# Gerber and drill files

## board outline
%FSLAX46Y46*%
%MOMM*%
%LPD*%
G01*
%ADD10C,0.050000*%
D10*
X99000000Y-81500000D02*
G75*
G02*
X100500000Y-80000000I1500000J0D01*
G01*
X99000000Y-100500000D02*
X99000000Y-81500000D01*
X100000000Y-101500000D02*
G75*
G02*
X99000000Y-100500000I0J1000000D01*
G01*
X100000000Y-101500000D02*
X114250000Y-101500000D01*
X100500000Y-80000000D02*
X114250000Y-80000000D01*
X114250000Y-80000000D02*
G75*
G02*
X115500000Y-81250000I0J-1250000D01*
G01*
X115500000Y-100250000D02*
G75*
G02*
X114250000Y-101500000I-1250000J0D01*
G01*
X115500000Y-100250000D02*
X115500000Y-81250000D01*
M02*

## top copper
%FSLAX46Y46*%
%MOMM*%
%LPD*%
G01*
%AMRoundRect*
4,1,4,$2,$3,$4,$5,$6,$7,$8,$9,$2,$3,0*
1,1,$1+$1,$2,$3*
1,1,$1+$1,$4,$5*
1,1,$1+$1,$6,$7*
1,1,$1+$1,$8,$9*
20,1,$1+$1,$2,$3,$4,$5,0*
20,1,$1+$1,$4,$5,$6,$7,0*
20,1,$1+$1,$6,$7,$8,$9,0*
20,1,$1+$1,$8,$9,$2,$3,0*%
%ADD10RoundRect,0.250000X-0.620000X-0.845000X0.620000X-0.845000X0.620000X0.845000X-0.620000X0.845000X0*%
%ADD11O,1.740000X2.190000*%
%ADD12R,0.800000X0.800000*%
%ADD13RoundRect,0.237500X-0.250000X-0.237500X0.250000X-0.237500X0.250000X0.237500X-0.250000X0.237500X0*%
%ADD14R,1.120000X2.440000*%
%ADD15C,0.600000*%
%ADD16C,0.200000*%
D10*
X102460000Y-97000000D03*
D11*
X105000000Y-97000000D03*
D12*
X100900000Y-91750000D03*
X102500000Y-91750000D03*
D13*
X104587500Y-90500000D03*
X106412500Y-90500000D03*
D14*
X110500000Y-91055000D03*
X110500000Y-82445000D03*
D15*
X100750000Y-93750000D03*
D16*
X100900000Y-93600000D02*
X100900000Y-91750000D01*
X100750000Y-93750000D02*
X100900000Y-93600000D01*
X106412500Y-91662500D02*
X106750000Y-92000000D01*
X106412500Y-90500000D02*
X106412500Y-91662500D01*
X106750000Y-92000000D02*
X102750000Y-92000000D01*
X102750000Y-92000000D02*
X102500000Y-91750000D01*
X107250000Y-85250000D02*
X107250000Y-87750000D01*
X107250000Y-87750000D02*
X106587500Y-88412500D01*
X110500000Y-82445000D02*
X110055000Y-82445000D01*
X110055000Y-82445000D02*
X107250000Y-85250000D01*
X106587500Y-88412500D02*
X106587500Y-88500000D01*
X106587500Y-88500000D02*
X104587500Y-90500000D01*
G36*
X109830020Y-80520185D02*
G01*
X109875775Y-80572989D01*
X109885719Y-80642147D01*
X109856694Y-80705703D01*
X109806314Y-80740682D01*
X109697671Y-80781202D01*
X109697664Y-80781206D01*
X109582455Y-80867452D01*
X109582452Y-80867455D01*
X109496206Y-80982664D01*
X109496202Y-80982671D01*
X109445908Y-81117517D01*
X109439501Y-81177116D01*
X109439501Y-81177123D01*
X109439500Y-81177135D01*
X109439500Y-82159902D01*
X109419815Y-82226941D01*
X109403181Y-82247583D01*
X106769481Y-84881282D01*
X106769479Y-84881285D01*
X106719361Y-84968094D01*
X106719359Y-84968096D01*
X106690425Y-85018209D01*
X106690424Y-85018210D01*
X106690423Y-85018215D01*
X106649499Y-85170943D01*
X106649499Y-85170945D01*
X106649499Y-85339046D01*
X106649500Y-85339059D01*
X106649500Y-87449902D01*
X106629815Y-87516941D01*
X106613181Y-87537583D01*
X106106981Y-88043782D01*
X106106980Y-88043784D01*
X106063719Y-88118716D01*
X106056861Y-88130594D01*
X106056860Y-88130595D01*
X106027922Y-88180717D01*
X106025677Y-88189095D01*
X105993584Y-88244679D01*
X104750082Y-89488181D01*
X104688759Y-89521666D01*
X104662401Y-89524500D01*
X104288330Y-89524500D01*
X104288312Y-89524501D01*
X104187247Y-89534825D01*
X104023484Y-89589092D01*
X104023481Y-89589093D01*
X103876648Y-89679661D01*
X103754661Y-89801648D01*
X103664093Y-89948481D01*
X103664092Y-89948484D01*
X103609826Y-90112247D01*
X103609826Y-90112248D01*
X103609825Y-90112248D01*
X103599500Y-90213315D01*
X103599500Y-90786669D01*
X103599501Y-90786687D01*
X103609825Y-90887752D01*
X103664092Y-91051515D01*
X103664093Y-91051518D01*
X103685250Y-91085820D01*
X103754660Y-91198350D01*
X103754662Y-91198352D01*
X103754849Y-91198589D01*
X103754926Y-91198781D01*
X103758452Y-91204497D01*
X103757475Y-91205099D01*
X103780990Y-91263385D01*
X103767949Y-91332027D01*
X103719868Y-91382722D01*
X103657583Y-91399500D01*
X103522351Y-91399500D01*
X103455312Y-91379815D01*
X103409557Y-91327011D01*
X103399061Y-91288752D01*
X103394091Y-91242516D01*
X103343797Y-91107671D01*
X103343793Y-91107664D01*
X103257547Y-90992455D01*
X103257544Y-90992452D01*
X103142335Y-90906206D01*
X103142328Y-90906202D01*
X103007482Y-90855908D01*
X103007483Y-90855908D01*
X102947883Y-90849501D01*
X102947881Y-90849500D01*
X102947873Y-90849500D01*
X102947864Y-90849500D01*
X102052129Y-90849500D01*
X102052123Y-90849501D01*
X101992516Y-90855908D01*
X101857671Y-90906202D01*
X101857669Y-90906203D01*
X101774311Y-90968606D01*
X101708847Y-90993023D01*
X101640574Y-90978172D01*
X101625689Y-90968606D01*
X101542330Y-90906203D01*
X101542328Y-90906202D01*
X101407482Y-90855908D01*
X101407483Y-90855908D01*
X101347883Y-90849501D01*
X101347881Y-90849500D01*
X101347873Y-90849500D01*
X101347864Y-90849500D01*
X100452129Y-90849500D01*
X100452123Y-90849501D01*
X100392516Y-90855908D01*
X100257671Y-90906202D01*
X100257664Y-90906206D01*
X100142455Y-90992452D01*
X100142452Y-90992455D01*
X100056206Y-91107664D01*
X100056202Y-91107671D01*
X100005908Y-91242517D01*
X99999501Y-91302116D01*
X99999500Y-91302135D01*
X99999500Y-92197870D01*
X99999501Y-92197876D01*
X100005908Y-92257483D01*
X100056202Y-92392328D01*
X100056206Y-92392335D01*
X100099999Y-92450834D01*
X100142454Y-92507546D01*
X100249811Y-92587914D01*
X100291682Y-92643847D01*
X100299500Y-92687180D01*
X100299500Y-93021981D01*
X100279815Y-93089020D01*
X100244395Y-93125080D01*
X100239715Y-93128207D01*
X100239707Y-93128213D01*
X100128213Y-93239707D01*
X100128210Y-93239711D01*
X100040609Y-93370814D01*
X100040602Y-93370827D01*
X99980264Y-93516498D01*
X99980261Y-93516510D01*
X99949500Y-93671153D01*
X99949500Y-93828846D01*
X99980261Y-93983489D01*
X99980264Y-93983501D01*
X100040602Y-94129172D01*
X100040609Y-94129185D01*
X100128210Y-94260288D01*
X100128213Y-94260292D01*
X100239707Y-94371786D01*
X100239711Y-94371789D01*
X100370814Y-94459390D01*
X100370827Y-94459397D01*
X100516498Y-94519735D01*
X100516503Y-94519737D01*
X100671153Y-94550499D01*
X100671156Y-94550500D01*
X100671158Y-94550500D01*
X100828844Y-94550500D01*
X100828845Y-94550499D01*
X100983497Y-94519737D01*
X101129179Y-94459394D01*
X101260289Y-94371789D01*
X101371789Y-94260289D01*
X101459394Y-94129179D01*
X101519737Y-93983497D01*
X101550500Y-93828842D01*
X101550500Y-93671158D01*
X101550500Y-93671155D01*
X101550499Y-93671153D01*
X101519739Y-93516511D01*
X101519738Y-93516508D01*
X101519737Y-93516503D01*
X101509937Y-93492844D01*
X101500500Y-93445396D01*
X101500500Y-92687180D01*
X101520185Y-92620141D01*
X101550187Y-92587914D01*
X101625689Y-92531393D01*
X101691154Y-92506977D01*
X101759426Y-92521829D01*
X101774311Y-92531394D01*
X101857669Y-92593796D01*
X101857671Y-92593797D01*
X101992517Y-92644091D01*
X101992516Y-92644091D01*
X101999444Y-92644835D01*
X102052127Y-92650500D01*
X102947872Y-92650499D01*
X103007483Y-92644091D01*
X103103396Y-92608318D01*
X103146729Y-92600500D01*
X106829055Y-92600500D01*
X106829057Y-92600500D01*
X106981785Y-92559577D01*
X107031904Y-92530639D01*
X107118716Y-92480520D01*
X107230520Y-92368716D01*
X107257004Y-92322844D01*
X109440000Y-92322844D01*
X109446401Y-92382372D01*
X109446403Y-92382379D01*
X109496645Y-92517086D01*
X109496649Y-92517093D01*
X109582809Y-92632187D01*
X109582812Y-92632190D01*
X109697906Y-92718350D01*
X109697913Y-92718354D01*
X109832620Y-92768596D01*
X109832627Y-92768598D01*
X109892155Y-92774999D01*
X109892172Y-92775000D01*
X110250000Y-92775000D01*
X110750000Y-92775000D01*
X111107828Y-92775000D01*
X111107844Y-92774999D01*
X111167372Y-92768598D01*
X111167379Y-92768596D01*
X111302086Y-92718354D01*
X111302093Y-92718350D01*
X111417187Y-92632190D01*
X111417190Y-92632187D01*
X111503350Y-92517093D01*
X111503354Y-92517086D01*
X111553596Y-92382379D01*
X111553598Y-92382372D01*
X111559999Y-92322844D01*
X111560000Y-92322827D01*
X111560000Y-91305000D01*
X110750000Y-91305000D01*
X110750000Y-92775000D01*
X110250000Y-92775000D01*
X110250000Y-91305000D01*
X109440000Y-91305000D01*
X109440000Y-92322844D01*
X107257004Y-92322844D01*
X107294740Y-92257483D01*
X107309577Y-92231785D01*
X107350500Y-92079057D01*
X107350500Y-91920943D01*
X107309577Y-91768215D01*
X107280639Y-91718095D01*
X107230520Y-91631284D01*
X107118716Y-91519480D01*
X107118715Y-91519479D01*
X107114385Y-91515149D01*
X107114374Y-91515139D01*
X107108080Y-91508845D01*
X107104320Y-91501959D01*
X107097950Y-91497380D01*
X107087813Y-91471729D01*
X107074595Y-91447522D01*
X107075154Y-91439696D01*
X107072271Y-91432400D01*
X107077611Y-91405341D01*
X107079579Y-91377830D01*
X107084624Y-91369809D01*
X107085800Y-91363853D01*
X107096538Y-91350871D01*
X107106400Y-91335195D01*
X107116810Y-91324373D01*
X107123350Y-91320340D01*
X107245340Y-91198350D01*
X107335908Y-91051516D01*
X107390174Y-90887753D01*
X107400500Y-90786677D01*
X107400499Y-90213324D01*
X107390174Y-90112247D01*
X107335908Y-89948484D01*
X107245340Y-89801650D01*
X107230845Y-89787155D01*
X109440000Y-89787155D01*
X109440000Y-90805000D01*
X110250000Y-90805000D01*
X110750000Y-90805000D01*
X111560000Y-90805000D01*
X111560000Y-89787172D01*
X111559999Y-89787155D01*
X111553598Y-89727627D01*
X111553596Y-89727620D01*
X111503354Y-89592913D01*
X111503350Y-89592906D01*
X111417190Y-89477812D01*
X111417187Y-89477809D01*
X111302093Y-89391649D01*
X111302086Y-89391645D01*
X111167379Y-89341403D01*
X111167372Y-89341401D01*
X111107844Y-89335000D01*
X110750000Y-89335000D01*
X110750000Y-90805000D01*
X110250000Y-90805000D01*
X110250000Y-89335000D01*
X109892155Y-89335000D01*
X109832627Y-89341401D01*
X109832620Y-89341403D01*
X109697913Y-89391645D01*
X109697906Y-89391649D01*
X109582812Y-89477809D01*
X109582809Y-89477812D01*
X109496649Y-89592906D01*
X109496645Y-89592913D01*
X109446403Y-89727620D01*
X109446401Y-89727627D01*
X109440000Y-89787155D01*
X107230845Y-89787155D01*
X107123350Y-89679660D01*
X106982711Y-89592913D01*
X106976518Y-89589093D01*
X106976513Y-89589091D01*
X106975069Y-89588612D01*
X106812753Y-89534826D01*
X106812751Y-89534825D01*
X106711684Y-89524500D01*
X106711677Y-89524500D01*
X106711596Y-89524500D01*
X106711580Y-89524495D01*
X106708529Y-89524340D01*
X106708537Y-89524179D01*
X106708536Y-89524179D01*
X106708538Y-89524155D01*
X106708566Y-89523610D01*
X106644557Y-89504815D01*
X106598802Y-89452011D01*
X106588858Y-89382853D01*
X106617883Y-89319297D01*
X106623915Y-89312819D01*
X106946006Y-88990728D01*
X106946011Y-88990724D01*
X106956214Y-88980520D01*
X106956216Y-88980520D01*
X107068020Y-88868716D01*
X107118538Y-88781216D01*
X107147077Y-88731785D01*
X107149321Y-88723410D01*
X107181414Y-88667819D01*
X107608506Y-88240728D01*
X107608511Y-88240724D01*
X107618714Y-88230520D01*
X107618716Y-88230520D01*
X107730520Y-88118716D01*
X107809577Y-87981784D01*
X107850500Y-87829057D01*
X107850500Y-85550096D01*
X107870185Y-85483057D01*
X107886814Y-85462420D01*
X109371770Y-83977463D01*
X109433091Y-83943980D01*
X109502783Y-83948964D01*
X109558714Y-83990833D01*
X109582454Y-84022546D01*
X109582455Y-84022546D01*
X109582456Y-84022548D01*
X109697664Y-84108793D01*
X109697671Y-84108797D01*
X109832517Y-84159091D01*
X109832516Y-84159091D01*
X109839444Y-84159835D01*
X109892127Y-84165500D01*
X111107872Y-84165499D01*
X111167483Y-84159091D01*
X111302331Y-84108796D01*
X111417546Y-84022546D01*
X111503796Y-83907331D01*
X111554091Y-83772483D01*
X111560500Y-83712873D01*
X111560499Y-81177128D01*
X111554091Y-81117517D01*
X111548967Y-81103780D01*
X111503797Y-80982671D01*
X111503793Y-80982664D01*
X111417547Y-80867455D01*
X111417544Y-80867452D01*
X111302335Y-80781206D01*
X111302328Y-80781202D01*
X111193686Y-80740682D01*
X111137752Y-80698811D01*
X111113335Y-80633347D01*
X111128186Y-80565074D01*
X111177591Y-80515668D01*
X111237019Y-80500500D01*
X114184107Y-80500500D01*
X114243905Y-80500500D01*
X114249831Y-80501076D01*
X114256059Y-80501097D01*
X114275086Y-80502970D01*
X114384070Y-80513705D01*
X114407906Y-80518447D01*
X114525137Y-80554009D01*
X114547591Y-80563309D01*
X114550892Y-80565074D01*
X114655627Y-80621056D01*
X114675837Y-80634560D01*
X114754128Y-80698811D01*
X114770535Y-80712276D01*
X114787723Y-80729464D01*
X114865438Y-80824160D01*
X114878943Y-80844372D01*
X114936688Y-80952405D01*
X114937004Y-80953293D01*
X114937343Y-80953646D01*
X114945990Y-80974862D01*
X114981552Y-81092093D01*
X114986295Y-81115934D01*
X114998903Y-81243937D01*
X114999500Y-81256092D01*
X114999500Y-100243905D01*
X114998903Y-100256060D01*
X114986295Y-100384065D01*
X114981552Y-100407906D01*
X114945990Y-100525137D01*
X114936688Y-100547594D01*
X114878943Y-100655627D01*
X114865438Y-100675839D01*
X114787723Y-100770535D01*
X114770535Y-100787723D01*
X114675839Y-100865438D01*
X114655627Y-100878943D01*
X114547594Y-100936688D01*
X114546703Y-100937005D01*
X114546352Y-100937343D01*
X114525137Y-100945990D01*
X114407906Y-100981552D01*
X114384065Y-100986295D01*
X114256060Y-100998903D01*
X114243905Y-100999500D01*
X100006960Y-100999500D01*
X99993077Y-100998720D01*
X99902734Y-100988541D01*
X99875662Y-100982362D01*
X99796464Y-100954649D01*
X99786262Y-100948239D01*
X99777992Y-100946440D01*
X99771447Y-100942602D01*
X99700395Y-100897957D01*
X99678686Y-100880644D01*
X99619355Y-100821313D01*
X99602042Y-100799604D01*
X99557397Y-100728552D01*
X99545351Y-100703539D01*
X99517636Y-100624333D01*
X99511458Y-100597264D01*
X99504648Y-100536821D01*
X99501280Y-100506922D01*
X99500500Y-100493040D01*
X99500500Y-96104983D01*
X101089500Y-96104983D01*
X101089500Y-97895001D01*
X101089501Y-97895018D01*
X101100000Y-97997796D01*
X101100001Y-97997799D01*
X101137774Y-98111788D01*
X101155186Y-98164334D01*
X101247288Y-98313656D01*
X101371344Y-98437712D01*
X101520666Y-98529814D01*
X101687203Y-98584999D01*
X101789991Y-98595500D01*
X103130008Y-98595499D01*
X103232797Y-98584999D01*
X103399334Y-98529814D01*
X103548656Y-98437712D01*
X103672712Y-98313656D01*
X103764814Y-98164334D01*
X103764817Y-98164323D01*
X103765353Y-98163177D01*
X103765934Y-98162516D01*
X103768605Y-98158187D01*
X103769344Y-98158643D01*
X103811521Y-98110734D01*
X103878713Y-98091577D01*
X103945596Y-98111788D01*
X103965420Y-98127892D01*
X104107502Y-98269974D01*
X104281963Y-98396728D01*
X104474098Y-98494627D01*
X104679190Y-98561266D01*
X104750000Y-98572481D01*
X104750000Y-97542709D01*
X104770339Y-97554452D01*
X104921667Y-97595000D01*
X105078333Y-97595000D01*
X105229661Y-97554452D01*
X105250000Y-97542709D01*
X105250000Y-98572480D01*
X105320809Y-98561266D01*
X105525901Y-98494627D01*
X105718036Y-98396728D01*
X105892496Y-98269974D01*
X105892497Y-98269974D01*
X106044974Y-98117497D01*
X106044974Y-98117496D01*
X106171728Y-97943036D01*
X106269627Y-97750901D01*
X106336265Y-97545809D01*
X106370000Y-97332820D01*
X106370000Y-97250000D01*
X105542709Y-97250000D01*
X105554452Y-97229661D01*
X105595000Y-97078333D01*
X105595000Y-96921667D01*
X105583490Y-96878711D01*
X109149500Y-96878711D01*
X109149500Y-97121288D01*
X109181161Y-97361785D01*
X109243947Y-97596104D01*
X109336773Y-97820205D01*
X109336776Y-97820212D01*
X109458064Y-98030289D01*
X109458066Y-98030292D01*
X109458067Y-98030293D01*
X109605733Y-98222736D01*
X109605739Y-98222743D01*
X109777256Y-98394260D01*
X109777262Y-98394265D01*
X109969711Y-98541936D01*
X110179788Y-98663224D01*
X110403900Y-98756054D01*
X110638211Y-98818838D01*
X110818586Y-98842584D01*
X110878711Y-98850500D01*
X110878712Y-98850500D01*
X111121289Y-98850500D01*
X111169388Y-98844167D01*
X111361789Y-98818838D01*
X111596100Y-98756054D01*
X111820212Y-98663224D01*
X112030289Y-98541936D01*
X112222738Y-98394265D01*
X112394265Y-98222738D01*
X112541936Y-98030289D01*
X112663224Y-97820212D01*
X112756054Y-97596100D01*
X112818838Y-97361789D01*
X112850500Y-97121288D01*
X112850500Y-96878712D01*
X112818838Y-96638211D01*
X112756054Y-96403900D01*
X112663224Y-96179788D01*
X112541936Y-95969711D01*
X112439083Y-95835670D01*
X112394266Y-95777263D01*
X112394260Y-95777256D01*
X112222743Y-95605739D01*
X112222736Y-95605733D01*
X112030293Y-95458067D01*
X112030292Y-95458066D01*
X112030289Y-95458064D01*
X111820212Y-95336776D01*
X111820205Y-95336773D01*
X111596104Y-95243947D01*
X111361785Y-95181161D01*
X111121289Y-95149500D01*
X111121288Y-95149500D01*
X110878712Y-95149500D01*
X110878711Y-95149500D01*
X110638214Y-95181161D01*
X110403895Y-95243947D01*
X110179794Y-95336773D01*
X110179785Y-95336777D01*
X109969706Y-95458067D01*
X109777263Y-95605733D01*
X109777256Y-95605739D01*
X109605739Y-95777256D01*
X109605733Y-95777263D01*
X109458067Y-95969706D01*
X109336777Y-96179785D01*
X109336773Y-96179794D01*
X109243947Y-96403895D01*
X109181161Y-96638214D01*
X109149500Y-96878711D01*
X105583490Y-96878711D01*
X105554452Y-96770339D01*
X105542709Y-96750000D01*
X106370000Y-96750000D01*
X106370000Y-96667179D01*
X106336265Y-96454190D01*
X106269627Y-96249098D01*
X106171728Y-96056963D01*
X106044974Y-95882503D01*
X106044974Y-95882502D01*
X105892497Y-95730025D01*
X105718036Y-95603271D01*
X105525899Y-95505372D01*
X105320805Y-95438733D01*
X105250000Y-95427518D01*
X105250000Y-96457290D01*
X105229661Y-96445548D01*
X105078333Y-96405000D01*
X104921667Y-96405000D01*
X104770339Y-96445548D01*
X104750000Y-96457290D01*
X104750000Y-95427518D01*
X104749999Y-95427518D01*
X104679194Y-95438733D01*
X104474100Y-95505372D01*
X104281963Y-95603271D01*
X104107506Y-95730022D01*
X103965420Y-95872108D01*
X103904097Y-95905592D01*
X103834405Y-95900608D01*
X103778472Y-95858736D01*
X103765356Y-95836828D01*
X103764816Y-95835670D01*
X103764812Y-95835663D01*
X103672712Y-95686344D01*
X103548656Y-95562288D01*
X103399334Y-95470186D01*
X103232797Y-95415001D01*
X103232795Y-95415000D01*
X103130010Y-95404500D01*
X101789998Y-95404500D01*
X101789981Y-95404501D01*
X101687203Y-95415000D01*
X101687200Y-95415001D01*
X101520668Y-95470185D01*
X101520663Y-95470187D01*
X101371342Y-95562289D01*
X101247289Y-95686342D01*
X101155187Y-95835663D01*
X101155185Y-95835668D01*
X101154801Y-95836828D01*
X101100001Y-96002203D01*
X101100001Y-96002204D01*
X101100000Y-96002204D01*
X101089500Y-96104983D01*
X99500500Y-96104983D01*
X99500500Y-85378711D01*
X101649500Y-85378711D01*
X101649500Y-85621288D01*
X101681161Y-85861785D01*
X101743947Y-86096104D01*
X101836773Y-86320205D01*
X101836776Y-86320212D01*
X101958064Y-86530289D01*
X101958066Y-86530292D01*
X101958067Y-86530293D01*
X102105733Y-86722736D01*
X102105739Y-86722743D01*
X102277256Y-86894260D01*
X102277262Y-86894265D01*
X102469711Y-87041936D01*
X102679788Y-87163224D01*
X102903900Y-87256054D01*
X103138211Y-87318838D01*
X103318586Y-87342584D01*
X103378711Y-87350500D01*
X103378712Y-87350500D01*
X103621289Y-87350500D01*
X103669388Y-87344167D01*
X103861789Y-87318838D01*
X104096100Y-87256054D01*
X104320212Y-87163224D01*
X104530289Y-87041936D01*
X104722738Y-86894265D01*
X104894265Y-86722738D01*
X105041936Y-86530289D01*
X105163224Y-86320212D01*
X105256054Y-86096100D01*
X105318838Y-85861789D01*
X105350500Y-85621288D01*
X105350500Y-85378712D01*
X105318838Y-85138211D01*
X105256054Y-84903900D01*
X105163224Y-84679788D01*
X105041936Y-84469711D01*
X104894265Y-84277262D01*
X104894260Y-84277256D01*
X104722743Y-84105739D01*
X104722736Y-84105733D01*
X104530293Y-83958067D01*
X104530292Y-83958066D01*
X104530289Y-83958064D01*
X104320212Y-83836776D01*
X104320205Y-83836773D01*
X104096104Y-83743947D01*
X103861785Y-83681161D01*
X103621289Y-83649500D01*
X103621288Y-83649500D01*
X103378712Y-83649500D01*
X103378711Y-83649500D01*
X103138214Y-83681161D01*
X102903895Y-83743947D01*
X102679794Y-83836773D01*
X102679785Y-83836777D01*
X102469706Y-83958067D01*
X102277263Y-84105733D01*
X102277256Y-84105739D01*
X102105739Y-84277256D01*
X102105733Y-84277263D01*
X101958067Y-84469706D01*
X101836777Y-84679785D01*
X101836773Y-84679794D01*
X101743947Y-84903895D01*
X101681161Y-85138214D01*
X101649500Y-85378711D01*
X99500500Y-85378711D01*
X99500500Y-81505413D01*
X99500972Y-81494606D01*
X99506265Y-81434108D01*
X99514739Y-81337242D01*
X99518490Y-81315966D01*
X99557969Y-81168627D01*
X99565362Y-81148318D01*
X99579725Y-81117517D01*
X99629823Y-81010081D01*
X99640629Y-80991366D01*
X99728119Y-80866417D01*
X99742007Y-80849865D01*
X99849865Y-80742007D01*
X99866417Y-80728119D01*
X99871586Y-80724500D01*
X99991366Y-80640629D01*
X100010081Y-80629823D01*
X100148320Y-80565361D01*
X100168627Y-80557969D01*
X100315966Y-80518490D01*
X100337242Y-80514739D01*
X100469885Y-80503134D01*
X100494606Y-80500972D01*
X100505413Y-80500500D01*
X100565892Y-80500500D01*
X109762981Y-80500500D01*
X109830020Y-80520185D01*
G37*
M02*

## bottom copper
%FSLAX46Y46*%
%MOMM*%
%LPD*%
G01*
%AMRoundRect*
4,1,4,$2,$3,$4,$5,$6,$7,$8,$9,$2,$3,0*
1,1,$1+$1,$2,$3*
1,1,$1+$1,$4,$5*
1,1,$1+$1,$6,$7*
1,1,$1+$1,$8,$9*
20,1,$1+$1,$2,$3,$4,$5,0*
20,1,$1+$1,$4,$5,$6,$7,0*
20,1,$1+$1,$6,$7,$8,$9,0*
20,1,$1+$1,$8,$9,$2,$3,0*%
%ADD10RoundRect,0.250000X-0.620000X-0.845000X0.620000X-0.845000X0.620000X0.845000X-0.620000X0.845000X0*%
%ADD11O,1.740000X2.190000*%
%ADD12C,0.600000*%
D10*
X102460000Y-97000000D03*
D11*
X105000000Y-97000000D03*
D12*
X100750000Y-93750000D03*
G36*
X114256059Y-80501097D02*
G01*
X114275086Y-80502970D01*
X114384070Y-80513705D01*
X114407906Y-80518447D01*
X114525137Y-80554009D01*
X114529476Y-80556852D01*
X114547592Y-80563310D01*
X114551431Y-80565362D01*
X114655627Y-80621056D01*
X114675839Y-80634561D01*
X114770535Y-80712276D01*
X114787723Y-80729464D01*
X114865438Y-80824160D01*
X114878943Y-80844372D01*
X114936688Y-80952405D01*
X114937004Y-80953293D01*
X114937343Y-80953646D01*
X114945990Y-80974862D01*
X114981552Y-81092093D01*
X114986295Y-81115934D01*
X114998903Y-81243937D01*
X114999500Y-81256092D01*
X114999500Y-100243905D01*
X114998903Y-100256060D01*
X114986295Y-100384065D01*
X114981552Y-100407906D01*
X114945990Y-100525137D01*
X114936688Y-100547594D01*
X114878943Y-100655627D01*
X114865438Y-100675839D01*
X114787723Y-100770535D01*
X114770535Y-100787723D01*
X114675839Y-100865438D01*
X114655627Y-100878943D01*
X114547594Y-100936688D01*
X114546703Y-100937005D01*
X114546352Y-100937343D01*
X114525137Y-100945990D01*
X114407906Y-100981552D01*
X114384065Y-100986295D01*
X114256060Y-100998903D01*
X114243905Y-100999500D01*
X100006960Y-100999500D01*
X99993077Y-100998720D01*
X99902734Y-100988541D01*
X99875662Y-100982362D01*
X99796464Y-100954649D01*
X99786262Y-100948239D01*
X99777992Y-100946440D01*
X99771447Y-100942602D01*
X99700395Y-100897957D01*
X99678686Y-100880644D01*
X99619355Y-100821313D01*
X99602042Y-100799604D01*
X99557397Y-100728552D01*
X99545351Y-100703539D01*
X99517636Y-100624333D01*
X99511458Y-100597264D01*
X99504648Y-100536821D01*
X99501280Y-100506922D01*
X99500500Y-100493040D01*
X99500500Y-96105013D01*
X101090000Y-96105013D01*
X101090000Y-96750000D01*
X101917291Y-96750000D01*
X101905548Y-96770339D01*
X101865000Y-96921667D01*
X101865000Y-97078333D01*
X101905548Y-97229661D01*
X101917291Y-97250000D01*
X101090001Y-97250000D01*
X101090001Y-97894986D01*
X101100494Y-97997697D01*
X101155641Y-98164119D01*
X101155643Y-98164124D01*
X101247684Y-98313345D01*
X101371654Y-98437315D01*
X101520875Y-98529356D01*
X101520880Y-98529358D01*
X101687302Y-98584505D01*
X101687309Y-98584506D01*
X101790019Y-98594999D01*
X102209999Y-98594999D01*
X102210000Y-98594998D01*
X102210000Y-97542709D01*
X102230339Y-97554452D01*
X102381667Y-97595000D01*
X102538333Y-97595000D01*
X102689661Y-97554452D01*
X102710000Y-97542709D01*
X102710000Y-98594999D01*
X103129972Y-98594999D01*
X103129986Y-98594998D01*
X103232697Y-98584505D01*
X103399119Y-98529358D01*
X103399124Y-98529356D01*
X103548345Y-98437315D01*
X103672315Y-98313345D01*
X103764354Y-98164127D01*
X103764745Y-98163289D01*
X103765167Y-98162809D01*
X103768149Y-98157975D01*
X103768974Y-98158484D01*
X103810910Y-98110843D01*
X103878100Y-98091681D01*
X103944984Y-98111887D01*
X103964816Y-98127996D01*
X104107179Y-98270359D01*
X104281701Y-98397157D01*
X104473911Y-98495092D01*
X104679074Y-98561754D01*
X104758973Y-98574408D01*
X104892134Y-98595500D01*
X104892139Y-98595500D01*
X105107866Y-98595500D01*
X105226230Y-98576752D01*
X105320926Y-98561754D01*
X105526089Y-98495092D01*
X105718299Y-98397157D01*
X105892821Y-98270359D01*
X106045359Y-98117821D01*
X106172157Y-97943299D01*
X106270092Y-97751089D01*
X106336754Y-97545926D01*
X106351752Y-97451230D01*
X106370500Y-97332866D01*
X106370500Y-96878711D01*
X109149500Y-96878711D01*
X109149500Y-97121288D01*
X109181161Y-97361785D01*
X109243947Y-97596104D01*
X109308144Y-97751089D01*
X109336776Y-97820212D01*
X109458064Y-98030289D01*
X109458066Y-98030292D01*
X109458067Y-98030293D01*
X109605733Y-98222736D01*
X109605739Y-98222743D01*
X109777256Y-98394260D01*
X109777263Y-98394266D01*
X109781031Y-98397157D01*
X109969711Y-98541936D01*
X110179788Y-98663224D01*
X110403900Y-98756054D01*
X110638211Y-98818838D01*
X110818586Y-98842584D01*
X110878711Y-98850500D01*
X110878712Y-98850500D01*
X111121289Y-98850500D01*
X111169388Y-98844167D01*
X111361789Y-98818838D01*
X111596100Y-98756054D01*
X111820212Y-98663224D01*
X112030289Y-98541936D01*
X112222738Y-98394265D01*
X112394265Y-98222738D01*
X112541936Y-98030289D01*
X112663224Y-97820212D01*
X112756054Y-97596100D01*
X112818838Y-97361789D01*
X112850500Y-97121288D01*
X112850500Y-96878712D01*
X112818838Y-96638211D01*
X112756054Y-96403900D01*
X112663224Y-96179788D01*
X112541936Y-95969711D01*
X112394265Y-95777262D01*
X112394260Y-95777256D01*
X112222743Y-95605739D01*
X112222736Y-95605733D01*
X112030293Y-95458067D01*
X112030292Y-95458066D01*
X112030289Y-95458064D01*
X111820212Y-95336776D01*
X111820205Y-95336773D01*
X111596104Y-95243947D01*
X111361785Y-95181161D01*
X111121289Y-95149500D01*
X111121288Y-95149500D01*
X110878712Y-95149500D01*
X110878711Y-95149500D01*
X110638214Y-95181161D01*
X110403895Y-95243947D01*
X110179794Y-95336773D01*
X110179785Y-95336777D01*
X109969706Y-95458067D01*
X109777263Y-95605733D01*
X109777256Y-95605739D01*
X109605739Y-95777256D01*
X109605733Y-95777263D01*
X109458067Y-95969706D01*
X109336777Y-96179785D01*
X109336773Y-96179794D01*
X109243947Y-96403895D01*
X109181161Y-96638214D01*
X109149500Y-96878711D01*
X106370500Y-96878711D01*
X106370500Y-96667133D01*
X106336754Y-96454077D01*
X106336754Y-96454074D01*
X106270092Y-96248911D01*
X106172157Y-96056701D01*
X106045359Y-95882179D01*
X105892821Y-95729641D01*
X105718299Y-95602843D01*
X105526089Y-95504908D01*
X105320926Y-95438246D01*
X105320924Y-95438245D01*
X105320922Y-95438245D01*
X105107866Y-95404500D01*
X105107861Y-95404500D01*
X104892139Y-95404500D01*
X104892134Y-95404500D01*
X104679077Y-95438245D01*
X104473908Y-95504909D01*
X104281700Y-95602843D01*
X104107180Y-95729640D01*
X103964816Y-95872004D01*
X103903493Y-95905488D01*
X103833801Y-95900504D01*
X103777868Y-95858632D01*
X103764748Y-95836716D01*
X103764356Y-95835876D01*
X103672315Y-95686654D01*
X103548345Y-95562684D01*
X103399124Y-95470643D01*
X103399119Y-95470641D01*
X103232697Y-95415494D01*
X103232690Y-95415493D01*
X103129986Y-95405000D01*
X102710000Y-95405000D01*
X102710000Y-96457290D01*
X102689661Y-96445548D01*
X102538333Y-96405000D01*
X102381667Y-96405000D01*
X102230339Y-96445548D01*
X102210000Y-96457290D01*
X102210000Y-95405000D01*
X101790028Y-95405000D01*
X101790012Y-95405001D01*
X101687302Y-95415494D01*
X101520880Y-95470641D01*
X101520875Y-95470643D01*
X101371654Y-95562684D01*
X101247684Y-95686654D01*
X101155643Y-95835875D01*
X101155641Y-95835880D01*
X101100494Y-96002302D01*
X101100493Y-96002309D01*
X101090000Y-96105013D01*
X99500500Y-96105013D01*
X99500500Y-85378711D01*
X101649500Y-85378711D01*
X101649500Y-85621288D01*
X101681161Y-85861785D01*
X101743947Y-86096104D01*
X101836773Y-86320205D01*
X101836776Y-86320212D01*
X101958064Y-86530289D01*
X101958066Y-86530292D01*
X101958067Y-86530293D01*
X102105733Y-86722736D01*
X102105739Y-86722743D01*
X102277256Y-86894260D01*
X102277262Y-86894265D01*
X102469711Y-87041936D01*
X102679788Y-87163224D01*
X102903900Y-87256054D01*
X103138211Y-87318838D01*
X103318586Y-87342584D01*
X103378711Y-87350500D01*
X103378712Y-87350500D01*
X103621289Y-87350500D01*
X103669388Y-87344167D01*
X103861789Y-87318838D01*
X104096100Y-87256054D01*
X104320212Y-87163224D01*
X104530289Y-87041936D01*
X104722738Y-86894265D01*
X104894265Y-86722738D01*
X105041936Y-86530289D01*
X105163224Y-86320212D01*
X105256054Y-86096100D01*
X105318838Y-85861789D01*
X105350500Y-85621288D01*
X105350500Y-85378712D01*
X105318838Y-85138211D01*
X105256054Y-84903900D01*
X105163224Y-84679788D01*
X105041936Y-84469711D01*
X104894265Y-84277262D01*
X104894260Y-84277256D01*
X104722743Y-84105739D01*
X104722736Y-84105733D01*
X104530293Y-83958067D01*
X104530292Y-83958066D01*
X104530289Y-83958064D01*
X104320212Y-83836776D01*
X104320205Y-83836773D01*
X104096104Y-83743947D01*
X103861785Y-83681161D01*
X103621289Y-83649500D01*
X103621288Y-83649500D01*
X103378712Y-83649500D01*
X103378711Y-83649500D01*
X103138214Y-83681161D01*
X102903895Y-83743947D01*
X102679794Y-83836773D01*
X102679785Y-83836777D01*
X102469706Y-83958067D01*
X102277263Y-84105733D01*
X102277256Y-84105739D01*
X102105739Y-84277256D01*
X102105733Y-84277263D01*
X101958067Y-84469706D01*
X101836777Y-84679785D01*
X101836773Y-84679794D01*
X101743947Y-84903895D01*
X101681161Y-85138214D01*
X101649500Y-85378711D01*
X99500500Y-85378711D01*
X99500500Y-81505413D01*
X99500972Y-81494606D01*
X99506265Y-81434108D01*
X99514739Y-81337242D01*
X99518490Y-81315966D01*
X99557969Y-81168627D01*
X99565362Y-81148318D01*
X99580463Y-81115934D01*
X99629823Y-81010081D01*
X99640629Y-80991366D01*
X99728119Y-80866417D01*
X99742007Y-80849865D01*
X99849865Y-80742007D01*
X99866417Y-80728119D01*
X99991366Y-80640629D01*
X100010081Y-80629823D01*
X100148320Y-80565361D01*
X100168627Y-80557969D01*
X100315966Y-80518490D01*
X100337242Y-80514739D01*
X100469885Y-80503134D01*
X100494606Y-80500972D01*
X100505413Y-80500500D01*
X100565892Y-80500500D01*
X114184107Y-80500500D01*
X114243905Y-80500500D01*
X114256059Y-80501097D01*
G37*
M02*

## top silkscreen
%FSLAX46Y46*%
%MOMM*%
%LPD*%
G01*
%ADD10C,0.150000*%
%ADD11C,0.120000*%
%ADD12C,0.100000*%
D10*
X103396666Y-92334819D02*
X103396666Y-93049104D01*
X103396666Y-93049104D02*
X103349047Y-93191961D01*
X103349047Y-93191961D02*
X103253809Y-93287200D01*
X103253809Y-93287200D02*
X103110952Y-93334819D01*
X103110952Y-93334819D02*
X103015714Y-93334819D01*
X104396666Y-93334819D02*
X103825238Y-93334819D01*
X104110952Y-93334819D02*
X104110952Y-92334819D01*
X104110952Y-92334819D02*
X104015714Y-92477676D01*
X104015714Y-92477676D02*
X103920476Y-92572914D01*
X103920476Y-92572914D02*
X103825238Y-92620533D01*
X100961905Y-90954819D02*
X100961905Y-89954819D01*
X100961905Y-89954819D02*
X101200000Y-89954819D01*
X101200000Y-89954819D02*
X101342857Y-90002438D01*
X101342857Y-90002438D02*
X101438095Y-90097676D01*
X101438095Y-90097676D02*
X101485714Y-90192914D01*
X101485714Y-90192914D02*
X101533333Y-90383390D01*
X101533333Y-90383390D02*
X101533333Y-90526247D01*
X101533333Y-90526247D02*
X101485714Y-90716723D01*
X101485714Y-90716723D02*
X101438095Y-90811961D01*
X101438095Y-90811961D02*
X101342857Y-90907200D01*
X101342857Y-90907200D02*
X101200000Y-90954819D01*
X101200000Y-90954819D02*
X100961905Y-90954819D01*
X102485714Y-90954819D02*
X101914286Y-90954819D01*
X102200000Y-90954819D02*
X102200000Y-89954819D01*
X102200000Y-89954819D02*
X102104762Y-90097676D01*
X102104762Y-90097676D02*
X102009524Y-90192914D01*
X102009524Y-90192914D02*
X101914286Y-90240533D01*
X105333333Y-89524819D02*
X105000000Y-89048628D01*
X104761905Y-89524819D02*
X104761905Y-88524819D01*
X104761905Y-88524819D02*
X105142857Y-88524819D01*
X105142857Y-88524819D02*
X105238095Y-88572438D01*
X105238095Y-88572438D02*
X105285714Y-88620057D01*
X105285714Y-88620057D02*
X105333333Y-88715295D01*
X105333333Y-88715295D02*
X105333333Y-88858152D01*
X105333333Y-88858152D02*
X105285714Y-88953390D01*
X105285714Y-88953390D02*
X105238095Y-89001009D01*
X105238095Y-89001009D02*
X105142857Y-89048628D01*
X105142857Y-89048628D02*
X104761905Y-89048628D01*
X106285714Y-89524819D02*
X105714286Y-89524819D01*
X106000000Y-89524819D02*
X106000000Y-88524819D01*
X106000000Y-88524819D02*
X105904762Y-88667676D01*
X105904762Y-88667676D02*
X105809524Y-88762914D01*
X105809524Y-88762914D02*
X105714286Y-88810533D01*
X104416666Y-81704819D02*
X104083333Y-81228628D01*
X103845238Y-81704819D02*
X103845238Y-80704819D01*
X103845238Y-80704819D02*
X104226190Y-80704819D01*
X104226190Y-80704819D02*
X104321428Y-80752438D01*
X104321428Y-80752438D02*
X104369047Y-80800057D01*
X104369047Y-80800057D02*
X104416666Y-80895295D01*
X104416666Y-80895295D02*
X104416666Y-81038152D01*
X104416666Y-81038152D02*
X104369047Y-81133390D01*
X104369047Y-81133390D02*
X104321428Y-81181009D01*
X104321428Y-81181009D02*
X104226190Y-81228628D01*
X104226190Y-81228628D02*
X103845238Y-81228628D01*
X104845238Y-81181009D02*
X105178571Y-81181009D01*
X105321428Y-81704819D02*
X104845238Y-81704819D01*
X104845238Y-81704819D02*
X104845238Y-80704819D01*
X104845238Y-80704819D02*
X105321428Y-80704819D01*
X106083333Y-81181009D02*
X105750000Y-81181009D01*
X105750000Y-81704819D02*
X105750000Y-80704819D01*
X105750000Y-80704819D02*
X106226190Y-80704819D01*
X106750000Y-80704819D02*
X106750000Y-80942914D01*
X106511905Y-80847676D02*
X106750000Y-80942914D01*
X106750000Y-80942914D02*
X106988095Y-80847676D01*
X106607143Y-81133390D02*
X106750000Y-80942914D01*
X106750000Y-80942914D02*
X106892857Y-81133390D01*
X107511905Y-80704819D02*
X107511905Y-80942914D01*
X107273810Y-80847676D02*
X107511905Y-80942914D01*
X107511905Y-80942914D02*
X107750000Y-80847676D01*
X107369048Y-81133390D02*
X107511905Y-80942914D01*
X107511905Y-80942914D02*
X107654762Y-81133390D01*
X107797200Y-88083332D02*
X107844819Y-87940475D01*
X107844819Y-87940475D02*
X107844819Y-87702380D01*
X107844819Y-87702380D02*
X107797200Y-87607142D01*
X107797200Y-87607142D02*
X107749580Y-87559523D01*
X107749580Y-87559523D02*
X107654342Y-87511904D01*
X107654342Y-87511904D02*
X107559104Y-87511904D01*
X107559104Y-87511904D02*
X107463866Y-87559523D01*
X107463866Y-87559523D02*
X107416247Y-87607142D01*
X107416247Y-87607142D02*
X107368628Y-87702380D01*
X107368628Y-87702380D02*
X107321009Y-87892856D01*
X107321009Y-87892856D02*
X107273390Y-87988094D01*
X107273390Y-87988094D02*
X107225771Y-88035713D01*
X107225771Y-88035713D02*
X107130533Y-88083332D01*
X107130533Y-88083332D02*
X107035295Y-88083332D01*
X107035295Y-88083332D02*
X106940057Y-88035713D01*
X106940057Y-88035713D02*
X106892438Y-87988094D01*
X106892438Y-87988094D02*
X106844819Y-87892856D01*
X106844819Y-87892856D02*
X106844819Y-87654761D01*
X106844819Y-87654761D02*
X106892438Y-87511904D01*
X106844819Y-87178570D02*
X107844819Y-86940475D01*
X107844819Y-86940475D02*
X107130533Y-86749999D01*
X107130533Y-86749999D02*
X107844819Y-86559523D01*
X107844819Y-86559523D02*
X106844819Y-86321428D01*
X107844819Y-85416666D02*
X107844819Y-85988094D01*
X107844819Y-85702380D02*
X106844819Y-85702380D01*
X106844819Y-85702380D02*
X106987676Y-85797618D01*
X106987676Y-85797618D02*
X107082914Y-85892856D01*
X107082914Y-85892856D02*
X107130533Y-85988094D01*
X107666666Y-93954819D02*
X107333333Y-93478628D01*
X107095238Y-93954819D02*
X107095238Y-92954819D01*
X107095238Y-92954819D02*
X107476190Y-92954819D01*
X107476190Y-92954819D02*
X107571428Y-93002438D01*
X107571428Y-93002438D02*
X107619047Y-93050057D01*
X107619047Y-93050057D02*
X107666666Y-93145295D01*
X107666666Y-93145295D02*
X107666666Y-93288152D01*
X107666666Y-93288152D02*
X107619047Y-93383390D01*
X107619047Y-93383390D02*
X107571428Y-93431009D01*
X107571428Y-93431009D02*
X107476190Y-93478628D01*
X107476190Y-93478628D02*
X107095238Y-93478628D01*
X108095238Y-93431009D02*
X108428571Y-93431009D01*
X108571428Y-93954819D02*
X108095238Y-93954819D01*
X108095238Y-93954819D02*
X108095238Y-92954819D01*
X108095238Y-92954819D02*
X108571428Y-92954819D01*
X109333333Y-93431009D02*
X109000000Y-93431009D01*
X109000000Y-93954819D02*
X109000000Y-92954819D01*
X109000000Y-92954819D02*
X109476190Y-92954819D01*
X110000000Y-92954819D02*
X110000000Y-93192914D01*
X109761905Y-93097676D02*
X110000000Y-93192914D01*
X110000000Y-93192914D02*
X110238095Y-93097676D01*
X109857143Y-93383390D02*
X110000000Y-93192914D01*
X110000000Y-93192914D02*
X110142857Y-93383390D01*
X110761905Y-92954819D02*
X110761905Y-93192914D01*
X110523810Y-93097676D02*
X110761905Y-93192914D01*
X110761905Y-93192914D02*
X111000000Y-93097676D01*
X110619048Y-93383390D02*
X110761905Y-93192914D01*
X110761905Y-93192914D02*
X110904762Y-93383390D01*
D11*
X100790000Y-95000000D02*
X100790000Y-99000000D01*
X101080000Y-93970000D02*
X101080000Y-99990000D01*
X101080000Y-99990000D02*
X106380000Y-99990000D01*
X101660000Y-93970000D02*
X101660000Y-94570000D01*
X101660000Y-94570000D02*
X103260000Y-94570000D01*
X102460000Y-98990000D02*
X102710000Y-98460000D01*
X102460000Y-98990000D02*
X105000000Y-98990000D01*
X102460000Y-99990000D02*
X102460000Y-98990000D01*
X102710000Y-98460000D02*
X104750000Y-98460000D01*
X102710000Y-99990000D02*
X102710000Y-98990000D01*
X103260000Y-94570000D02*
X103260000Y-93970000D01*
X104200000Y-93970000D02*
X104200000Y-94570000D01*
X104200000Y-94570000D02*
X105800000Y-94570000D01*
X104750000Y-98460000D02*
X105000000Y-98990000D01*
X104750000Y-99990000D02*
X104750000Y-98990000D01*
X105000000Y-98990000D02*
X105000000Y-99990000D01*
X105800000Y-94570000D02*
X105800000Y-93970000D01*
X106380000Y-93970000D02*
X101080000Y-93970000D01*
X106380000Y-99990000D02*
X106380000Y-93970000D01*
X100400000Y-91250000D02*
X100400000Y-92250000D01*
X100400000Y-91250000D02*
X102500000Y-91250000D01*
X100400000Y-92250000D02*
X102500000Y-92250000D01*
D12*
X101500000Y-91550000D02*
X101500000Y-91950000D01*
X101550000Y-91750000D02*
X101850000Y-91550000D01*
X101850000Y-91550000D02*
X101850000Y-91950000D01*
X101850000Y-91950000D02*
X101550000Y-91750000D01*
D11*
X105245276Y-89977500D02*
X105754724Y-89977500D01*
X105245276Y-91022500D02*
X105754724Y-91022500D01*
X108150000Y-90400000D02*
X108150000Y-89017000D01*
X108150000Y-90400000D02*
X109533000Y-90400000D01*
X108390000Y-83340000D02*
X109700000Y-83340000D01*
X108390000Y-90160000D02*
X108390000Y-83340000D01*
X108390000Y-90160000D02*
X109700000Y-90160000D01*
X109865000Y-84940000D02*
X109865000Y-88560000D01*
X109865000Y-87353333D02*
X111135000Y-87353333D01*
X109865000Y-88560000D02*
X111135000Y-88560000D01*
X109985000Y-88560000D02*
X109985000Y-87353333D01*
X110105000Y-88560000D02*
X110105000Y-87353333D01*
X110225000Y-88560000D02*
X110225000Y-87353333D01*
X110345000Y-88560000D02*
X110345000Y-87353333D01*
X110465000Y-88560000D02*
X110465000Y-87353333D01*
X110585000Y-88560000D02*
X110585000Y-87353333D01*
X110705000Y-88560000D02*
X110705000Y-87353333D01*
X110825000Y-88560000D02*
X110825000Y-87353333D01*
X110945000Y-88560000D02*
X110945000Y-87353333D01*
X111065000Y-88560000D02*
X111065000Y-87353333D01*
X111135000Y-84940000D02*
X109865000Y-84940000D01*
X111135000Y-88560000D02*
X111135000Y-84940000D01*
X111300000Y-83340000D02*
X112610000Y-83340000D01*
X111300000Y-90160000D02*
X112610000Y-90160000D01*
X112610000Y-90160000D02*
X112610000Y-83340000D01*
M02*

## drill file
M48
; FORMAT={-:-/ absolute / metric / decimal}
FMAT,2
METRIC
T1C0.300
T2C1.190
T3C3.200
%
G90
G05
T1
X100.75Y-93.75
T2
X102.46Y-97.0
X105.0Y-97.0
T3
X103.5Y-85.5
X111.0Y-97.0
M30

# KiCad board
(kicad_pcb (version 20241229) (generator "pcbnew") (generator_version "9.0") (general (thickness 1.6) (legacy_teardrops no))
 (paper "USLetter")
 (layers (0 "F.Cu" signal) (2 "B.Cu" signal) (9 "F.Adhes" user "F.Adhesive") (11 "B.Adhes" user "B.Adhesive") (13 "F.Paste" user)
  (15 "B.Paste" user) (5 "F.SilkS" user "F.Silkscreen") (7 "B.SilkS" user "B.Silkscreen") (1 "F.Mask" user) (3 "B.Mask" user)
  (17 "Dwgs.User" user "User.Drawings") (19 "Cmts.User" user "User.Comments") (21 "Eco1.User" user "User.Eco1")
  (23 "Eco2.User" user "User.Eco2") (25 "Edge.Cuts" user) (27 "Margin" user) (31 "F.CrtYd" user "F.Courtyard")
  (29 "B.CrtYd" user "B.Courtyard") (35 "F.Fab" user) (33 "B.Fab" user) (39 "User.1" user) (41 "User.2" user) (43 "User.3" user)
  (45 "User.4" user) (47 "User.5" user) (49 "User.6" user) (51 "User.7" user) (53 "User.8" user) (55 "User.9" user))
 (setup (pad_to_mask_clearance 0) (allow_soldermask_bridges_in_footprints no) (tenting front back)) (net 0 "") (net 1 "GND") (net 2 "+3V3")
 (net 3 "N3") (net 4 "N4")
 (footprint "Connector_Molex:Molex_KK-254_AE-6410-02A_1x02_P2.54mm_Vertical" (layer "F.Cu") (at 102.46 97)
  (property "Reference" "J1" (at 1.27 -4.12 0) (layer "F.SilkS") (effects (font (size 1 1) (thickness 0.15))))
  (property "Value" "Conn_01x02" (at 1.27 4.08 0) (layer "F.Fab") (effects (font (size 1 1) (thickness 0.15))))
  (fp_line (start -1.67 -2) (end -1.67 2) (stroke (width 0.12) (type solid)) (layer "F.SilkS"))
  (fp_line (start -1.38 -3.03) (end -1.38 2.99) (stroke (width 0.12) (type solid)) (layer "F.SilkS"))
  (fp_line (start -1.38 2.99) (end 3.92 2.99) (stroke (width 0.12) (type solid)) (layer "F.SilkS"))
  (fp_line (start -0.8 -3.03) (end -0.8 -2.43) (stroke (width 0.12) (type solid)) (layer "F.SilkS"))
  (fp_line (start -0.8 -2.43) (end 0.8 -2.43) (stroke (width 0.12) (type solid)) (layer "F.SilkS"))
  (fp_line (start 0 1.99) (end 0.25 1.46) (stroke (width 0.12) (type solid)) (layer "F.SilkS"))
  (fp_line (start 0 1.99) (end 2.54 1.99) (stroke (width 0.12) (type solid)) (layer "F.SilkS"))
  (fp_line (start 0 2.99) (end 0 1.99) (stroke (width 0.12) (type solid)) (layer "F.SilkS"))
  (fp_line (start 0.25 1.46) (end 2.29 1.46) (stroke (width 0.12) (type solid)) (layer "F.SilkS"))
  (fp_line (start 0.25 2.99) (end 0.25 1.99) (stroke (width 0.12) (type solid)) (layer "F.SilkS"))
  (fp_line (start 0.8 -2.43) (end 0.8 -3.03) (stroke (width 0.12) (type solid)) (layer "F.SilkS"))
  (fp_line (start 1.74 -3.03) (end 1.74 -2.43) (stroke (width 0.12) (type solid)) (layer "F.SilkS"))
  (fp_line (start 1.74 -2.43) (end 3.34 -2.43) (stroke (width 0.12) (type solid)) (layer "F.SilkS"))
  (fp_line (start 2.29 1.46) (end 2.54 1.99) (stroke (width 0.12) (type solid)) (layer "F.SilkS"))
  (fp_line (start 2.29 2.99) (end 2.29 1.99) (stroke (width 0.12) (type solid)) (layer "F.SilkS"))
  (fp_line (start 2.54 1.99) (end 2.54 2.99) (stroke (width 0.12) (type solid)) (layer "F.SilkS"))
  (fp_line (start 3.34 -2.43) (end 3.34 -3.03) (stroke (width 0.12) (type solid)) (layer "F.SilkS"))
  (fp_line (start 3.92 -3.03) (end -1.38 -3.03) (stroke (width 0.12) (type solid)) (layer "F.SilkS"))
  (fp_line (start 3.92 2.99) (end 3.92 -3.03) (stroke (width 0.12) (type solid)) (layer "F.SilkS"))
  (pad "1" thru_hole roundrect (at 0 0) (size 1.74 2.19) (drill 1.19) (layers "*.Cu" "*.Mask") (remove_unused_layers no)
   (roundrect_rratio 0.143678) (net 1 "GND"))
  (pad "2" thru_hole oval (at 2.54 0) (size 1.74 2.19) (drill 1.19) (layers "*.Cu" "*.Mask") (remove_unused_layers no) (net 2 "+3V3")))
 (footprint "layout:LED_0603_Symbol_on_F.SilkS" (layer "F.Cu") (at 101.7 91.75)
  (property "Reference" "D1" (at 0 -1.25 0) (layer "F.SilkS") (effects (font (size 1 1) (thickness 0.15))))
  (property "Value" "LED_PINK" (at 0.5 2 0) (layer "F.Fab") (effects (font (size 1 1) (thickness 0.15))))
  (fp_line (start -1.3 -0.5) (end -1.3 0.5) (stroke (width 0.12) (type solid)) (layer "F.SilkS"))
  (fp_line (start -1.3 -0.5) (end 0.8 -0.5) (stroke (width 0.12) (type solid)) (layer "F.SilkS"))
  (fp_line (start -1.3 0.5) (end 0.8 0.5) (stroke (width 0.12) (type solid)) (layer "F.SilkS"))
  (fp_line (start -0.2 -0.2) (end -0.2 0.2) (stroke (width 0.1) (type solid)) (layer "F.SilkS"))
  (fp_line (start -0.15 0) (end 0.15 -0.2) (stroke (width 0.1) (type solid)) (layer "F.SilkS"))
  (fp_line (start 0.15 -0.2) (end 0.15 0.2) (stroke (width 0.1) (type solid)) (layer "F.SilkS"))
  (fp_line (start 0.15 0.2) (end -0.15 0) (stroke (width 0.1) (type solid)) (layer "F.SilkS"))
  (pad "1" smd rect (at -0.8 0 180) (size 0.8 0.8) (layers "F.Cu" "F.Mask" "F.Paste") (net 1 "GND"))
  (pad "2" smd rect (at 0.8 0 180) (size 0.8 0.8) (layers "F.Cu" "F.Mask" "F.Paste") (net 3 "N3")))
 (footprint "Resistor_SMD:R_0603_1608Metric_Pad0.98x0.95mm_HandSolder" (layer "F.Cu") (at 105.5 90.5)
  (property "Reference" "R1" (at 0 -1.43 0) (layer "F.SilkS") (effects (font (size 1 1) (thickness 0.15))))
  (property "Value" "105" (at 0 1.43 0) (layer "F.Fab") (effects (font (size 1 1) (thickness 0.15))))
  (fp_line (start -0.254724 -0.5225) (end 0.254724 -0.5225) (stroke (width 0.12) (type solid)) (layer "F.SilkS"))
  (fp_line (start -0.254724 0.5225) (end 0.254724 0.5225) (stroke (width 0.12) (type solid)) (layer "F.SilkS"))
  (pad "1" smd roundrect (at -0.9125 0) (size 0.975 0.95) (layers "F.Cu" "F.Mask" "F.Paste") (roundrect_rratio 0.25) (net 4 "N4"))
  (pad "2" smd roundrect (at 0.9125 0) (size 0.975 0.95) (layers "F.Cu" "F.Mask" "F.Paste") (roundrect_rratio 0.25) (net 3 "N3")))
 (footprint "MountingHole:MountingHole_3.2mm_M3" (layer "F.Cu") (at 103.5 85.5)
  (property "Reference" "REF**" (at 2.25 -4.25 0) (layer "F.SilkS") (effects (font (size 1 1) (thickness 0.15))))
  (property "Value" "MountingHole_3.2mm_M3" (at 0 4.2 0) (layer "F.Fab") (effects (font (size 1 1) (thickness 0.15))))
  (pad "" np_thru_hole circle (at 0 0) (size 3.2 3.2) (drill 3.2) (layers "*.Cu" "*.Mask")))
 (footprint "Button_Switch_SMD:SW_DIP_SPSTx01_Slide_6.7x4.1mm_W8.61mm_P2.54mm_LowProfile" (layer "F.Cu") (at 110.5 86.75 90)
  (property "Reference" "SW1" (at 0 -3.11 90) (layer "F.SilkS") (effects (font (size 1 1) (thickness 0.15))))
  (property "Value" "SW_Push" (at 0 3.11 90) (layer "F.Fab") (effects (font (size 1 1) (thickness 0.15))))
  (fp_line (start -3.65 -2.35) (end -2.267 -2.35) (stroke (width 0.12) (type solid)) (layer "F.SilkS"))
  (fp_line (start -3.65 -2.35) (end -3.65 -0.967) (stroke (width 0.12) (type solid)) (layer "F.SilkS"))
  (fp_line (start 3.41 -2.11) (end 3.41 -0.8) (stroke (width 0.12) (type solid)) (layer "F.SilkS"))
  (fp_line (start -3.41 -2.11) (end 3.41 -2.11) (stroke (width 0.12) (type solid)) (layer "F.SilkS"))
  (fp_line (start -3.41 -2.11) (end -3.41 -0.8) (stroke (width 0.12) (type solid)) (layer "F.SilkS"))
  (fp_line (start 1.81 -0.635) (end -1.81 -0.635) (stroke (width 0.12) (type solid)) (layer "F.SilkS"))
  (fp_line (start -0.603333 -0.635) (end -0.603333 0.635) (stroke (width 0.12) (type solid)) (layer "F.SilkS"))
  (fp_line (start -1.81 -0.635) (end -1.81 0.635) (stroke (width 0.12) (type solid)) (layer "F.SilkS"))
  (fp_line (start -1.81 -0.515) (end -0.603333 -0.515) (stroke (width 0.12) (type solid)) (layer "F.SilkS"))
  (fp_line (start -1.81 -0.395) (end -0.603333 -0.395) (stroke (width 0.12) (type solid)) (layer "F.SilkS"))
  (fp_line (start -1.81 -0.275) (end -0.603333 -0.275) (stroke (width 0.12) (type solid)) (layer "F.SilkS"))
  (fp_line (start -1.81 -0.155) (end -0.603333 -0.155) (stroke (width 0.12) (type solid)) (layer "F.SilkS"))
  (fp_line (start -1.81 -0.035) (end -0.603333 -0.035) (stroke (width 0.12) (type solid)) (layer "F.SilkS"))
  (fp_line (start -1.81 0.085) (end -0.603333 0.085) (stroke (width 0.12) (type solid)) (layer "F.SilkS"))
  (fp_line (start -1.81 0.205) (end -0.603333 0.205) (stroke (width 0.12) (type solid)) (layer "F.SilkS"))
  (fp_line (start -1.81 0.325) (end -0.603333 0.325) (stroke (width 0.12) (type solid)) (layer "F.SilkS"))
  (fp_line (start -1.81 0.445) (end -0.603333 0.445) (stroke (width 0.12) (type solid)) (layer "F.SilkS"))
  (fp_line (start -1.81 0.565) (end -0.603333 0.565) (stroke (width 0.12) (type solid)) (layer "F.SilkS"))
  (fp_line (start 1.81 0.635) (end 1.81 -0.635) (stroke (width 0.12) (type solid)) (layer "F.SilkS"))
  (fp_line (start -1.81 0.635) (end 1.81 0.635) (stroke (width 0.12) (type solid)) (layer "F.SilkS"))
  (fp_line (start 3.41 0.8) (end 3.41 2.11) (stroke (width 0.12) (type solid)) (layer "F.SilkS"))
  (fp_line (start -3.41 0.8) (end -3.41 2.11) (stroke (width 0.12) (type solid)) (layer "F.SilkS"))
  (fp_line (start -3.41 2.11) (end 3.41 2.11) (stroke (width 0.12) (type solid)) (layer "F.SilkS"))
  (pad "1" smd rect (at -4.305 0 90) (size 2.44 1.12) (layers "F.Cu" "F.Mask" "F.Paste") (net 2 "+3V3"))
  (pad "2" smd rect (at 4.305 0 90) (size 2.44 1.12) (layers "F.Cu" "F.Mask" "F.Paste") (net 4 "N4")))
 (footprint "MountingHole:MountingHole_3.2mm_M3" (layer "F.Cu") (at 111 97)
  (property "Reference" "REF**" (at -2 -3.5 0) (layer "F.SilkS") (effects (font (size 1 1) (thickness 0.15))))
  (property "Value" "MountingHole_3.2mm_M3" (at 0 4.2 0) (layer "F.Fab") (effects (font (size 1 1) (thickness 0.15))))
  (pad "" np_thru_hole circle (at 0 0) (size 3.2 3.2) (drill 3.2) (layers "*.Cu" "*.Mask")))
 (gr_arc (start 99 81.5) (mid 99.43934 80.43934) (end 100.5 80) (stroke (width 0.05) (type default)) (layer "Edge.Cuts"))
 (gr_line (start 99 100.5) (end 99 81.5) (stroke (width 0.05) (type default)) (layer "Edge.Cuts"))
 (gr_arc (start 100 101.5) (mid 99.292893 101.207107) (end 99 100.5) (stroke (width 0.05) (type default)) (layer "Edge.Cuts"))
 (gr_line (start 100 101.5) (end 114.25 101.5) (stroke (width 0.05) (type default)) (layer "Edge.Cuts"))
 (gr_line (start 100.5 80) (end 114.25 80) (stroke (width 0.05) (type default)) (layer "Edge.Cuts"))
 (gr_arc (start 114.25 80) (mid 115.133883 80.366117) (end 115.5 81.25) (stroke (width 0.05) (type default)) (layer "Edge.Cuts"))
 (gr_arc (start 115.5 100.25) (mid 115.133883 101.133883) (end 114.25 101.5) (stroke (width 0.05) (type default)) (layer "Edge.Cuts"))
 (gr_line (start 115.5 100.25) (end 115.5 81.25) (stroke (width 0.05) (type default)) (layer "Edge.Cuts"))
 (segment (start 100.9 93.6) (end 100.9 91.75) (width 0.2) (layer "F.Cu") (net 1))
 (segment (start 100.75 93.75) (end 100.9 93.6) (width 0.2) (layer "F.Cu") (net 1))
 (via (at 100.75 93.75) (size 0.6) (drill 0.3) (layers "F.Cu" "B.Cu") (free yes) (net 1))
 (segment (start 106.4125 91.6625) (end 106.75 92) (width 0.2) (layer "F.Cu") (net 3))
 (segment (start 106.4125 90.5) (end 106.4125 91.6625) (width 0.2) (layer "F.Cu") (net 3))
 (segment (start 106.75 92) (end 102.75 92) (width 0.2) (layer "F.Cu") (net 3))
 (segment (start 102.75 92) (end 102.5 91.75) (width 0.2) (layer "F.Cu") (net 3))
 (segment (start 107.25 85.25) (end 107.25 87.75) (width 0.2) (layer "F.Cu") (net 4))
 (segment (start 107.25 87.75) (end 106.5875 88.4125) (width 0.2) (layer "F.Cu") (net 4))
 (segment (start 110.5 82.445) (end 110.055 82.445) (width 0.2) (layer "F.Cu") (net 4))
 (segment (start 110.055 82.445) (end 107.25 85.25) (width 0.2) (layer "F.Cu") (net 4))
 (segment (start 106.5875 88.4125) (end 106.5875 88.5) (width 0.2) (layer "F.Cu") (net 4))
 (segment (start 106.5875 88.5) (end 104.5875 90.5) (width 0.2) (layer "F.Cu") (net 4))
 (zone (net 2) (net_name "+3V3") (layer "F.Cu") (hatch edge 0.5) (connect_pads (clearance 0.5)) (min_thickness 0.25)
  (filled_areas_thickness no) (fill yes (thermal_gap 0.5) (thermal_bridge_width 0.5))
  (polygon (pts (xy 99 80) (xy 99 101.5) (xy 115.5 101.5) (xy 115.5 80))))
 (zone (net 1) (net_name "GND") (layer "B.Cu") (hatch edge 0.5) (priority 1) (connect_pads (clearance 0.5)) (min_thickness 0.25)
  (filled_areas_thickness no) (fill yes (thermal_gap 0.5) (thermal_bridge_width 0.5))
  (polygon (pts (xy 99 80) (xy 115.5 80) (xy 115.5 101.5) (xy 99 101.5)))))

